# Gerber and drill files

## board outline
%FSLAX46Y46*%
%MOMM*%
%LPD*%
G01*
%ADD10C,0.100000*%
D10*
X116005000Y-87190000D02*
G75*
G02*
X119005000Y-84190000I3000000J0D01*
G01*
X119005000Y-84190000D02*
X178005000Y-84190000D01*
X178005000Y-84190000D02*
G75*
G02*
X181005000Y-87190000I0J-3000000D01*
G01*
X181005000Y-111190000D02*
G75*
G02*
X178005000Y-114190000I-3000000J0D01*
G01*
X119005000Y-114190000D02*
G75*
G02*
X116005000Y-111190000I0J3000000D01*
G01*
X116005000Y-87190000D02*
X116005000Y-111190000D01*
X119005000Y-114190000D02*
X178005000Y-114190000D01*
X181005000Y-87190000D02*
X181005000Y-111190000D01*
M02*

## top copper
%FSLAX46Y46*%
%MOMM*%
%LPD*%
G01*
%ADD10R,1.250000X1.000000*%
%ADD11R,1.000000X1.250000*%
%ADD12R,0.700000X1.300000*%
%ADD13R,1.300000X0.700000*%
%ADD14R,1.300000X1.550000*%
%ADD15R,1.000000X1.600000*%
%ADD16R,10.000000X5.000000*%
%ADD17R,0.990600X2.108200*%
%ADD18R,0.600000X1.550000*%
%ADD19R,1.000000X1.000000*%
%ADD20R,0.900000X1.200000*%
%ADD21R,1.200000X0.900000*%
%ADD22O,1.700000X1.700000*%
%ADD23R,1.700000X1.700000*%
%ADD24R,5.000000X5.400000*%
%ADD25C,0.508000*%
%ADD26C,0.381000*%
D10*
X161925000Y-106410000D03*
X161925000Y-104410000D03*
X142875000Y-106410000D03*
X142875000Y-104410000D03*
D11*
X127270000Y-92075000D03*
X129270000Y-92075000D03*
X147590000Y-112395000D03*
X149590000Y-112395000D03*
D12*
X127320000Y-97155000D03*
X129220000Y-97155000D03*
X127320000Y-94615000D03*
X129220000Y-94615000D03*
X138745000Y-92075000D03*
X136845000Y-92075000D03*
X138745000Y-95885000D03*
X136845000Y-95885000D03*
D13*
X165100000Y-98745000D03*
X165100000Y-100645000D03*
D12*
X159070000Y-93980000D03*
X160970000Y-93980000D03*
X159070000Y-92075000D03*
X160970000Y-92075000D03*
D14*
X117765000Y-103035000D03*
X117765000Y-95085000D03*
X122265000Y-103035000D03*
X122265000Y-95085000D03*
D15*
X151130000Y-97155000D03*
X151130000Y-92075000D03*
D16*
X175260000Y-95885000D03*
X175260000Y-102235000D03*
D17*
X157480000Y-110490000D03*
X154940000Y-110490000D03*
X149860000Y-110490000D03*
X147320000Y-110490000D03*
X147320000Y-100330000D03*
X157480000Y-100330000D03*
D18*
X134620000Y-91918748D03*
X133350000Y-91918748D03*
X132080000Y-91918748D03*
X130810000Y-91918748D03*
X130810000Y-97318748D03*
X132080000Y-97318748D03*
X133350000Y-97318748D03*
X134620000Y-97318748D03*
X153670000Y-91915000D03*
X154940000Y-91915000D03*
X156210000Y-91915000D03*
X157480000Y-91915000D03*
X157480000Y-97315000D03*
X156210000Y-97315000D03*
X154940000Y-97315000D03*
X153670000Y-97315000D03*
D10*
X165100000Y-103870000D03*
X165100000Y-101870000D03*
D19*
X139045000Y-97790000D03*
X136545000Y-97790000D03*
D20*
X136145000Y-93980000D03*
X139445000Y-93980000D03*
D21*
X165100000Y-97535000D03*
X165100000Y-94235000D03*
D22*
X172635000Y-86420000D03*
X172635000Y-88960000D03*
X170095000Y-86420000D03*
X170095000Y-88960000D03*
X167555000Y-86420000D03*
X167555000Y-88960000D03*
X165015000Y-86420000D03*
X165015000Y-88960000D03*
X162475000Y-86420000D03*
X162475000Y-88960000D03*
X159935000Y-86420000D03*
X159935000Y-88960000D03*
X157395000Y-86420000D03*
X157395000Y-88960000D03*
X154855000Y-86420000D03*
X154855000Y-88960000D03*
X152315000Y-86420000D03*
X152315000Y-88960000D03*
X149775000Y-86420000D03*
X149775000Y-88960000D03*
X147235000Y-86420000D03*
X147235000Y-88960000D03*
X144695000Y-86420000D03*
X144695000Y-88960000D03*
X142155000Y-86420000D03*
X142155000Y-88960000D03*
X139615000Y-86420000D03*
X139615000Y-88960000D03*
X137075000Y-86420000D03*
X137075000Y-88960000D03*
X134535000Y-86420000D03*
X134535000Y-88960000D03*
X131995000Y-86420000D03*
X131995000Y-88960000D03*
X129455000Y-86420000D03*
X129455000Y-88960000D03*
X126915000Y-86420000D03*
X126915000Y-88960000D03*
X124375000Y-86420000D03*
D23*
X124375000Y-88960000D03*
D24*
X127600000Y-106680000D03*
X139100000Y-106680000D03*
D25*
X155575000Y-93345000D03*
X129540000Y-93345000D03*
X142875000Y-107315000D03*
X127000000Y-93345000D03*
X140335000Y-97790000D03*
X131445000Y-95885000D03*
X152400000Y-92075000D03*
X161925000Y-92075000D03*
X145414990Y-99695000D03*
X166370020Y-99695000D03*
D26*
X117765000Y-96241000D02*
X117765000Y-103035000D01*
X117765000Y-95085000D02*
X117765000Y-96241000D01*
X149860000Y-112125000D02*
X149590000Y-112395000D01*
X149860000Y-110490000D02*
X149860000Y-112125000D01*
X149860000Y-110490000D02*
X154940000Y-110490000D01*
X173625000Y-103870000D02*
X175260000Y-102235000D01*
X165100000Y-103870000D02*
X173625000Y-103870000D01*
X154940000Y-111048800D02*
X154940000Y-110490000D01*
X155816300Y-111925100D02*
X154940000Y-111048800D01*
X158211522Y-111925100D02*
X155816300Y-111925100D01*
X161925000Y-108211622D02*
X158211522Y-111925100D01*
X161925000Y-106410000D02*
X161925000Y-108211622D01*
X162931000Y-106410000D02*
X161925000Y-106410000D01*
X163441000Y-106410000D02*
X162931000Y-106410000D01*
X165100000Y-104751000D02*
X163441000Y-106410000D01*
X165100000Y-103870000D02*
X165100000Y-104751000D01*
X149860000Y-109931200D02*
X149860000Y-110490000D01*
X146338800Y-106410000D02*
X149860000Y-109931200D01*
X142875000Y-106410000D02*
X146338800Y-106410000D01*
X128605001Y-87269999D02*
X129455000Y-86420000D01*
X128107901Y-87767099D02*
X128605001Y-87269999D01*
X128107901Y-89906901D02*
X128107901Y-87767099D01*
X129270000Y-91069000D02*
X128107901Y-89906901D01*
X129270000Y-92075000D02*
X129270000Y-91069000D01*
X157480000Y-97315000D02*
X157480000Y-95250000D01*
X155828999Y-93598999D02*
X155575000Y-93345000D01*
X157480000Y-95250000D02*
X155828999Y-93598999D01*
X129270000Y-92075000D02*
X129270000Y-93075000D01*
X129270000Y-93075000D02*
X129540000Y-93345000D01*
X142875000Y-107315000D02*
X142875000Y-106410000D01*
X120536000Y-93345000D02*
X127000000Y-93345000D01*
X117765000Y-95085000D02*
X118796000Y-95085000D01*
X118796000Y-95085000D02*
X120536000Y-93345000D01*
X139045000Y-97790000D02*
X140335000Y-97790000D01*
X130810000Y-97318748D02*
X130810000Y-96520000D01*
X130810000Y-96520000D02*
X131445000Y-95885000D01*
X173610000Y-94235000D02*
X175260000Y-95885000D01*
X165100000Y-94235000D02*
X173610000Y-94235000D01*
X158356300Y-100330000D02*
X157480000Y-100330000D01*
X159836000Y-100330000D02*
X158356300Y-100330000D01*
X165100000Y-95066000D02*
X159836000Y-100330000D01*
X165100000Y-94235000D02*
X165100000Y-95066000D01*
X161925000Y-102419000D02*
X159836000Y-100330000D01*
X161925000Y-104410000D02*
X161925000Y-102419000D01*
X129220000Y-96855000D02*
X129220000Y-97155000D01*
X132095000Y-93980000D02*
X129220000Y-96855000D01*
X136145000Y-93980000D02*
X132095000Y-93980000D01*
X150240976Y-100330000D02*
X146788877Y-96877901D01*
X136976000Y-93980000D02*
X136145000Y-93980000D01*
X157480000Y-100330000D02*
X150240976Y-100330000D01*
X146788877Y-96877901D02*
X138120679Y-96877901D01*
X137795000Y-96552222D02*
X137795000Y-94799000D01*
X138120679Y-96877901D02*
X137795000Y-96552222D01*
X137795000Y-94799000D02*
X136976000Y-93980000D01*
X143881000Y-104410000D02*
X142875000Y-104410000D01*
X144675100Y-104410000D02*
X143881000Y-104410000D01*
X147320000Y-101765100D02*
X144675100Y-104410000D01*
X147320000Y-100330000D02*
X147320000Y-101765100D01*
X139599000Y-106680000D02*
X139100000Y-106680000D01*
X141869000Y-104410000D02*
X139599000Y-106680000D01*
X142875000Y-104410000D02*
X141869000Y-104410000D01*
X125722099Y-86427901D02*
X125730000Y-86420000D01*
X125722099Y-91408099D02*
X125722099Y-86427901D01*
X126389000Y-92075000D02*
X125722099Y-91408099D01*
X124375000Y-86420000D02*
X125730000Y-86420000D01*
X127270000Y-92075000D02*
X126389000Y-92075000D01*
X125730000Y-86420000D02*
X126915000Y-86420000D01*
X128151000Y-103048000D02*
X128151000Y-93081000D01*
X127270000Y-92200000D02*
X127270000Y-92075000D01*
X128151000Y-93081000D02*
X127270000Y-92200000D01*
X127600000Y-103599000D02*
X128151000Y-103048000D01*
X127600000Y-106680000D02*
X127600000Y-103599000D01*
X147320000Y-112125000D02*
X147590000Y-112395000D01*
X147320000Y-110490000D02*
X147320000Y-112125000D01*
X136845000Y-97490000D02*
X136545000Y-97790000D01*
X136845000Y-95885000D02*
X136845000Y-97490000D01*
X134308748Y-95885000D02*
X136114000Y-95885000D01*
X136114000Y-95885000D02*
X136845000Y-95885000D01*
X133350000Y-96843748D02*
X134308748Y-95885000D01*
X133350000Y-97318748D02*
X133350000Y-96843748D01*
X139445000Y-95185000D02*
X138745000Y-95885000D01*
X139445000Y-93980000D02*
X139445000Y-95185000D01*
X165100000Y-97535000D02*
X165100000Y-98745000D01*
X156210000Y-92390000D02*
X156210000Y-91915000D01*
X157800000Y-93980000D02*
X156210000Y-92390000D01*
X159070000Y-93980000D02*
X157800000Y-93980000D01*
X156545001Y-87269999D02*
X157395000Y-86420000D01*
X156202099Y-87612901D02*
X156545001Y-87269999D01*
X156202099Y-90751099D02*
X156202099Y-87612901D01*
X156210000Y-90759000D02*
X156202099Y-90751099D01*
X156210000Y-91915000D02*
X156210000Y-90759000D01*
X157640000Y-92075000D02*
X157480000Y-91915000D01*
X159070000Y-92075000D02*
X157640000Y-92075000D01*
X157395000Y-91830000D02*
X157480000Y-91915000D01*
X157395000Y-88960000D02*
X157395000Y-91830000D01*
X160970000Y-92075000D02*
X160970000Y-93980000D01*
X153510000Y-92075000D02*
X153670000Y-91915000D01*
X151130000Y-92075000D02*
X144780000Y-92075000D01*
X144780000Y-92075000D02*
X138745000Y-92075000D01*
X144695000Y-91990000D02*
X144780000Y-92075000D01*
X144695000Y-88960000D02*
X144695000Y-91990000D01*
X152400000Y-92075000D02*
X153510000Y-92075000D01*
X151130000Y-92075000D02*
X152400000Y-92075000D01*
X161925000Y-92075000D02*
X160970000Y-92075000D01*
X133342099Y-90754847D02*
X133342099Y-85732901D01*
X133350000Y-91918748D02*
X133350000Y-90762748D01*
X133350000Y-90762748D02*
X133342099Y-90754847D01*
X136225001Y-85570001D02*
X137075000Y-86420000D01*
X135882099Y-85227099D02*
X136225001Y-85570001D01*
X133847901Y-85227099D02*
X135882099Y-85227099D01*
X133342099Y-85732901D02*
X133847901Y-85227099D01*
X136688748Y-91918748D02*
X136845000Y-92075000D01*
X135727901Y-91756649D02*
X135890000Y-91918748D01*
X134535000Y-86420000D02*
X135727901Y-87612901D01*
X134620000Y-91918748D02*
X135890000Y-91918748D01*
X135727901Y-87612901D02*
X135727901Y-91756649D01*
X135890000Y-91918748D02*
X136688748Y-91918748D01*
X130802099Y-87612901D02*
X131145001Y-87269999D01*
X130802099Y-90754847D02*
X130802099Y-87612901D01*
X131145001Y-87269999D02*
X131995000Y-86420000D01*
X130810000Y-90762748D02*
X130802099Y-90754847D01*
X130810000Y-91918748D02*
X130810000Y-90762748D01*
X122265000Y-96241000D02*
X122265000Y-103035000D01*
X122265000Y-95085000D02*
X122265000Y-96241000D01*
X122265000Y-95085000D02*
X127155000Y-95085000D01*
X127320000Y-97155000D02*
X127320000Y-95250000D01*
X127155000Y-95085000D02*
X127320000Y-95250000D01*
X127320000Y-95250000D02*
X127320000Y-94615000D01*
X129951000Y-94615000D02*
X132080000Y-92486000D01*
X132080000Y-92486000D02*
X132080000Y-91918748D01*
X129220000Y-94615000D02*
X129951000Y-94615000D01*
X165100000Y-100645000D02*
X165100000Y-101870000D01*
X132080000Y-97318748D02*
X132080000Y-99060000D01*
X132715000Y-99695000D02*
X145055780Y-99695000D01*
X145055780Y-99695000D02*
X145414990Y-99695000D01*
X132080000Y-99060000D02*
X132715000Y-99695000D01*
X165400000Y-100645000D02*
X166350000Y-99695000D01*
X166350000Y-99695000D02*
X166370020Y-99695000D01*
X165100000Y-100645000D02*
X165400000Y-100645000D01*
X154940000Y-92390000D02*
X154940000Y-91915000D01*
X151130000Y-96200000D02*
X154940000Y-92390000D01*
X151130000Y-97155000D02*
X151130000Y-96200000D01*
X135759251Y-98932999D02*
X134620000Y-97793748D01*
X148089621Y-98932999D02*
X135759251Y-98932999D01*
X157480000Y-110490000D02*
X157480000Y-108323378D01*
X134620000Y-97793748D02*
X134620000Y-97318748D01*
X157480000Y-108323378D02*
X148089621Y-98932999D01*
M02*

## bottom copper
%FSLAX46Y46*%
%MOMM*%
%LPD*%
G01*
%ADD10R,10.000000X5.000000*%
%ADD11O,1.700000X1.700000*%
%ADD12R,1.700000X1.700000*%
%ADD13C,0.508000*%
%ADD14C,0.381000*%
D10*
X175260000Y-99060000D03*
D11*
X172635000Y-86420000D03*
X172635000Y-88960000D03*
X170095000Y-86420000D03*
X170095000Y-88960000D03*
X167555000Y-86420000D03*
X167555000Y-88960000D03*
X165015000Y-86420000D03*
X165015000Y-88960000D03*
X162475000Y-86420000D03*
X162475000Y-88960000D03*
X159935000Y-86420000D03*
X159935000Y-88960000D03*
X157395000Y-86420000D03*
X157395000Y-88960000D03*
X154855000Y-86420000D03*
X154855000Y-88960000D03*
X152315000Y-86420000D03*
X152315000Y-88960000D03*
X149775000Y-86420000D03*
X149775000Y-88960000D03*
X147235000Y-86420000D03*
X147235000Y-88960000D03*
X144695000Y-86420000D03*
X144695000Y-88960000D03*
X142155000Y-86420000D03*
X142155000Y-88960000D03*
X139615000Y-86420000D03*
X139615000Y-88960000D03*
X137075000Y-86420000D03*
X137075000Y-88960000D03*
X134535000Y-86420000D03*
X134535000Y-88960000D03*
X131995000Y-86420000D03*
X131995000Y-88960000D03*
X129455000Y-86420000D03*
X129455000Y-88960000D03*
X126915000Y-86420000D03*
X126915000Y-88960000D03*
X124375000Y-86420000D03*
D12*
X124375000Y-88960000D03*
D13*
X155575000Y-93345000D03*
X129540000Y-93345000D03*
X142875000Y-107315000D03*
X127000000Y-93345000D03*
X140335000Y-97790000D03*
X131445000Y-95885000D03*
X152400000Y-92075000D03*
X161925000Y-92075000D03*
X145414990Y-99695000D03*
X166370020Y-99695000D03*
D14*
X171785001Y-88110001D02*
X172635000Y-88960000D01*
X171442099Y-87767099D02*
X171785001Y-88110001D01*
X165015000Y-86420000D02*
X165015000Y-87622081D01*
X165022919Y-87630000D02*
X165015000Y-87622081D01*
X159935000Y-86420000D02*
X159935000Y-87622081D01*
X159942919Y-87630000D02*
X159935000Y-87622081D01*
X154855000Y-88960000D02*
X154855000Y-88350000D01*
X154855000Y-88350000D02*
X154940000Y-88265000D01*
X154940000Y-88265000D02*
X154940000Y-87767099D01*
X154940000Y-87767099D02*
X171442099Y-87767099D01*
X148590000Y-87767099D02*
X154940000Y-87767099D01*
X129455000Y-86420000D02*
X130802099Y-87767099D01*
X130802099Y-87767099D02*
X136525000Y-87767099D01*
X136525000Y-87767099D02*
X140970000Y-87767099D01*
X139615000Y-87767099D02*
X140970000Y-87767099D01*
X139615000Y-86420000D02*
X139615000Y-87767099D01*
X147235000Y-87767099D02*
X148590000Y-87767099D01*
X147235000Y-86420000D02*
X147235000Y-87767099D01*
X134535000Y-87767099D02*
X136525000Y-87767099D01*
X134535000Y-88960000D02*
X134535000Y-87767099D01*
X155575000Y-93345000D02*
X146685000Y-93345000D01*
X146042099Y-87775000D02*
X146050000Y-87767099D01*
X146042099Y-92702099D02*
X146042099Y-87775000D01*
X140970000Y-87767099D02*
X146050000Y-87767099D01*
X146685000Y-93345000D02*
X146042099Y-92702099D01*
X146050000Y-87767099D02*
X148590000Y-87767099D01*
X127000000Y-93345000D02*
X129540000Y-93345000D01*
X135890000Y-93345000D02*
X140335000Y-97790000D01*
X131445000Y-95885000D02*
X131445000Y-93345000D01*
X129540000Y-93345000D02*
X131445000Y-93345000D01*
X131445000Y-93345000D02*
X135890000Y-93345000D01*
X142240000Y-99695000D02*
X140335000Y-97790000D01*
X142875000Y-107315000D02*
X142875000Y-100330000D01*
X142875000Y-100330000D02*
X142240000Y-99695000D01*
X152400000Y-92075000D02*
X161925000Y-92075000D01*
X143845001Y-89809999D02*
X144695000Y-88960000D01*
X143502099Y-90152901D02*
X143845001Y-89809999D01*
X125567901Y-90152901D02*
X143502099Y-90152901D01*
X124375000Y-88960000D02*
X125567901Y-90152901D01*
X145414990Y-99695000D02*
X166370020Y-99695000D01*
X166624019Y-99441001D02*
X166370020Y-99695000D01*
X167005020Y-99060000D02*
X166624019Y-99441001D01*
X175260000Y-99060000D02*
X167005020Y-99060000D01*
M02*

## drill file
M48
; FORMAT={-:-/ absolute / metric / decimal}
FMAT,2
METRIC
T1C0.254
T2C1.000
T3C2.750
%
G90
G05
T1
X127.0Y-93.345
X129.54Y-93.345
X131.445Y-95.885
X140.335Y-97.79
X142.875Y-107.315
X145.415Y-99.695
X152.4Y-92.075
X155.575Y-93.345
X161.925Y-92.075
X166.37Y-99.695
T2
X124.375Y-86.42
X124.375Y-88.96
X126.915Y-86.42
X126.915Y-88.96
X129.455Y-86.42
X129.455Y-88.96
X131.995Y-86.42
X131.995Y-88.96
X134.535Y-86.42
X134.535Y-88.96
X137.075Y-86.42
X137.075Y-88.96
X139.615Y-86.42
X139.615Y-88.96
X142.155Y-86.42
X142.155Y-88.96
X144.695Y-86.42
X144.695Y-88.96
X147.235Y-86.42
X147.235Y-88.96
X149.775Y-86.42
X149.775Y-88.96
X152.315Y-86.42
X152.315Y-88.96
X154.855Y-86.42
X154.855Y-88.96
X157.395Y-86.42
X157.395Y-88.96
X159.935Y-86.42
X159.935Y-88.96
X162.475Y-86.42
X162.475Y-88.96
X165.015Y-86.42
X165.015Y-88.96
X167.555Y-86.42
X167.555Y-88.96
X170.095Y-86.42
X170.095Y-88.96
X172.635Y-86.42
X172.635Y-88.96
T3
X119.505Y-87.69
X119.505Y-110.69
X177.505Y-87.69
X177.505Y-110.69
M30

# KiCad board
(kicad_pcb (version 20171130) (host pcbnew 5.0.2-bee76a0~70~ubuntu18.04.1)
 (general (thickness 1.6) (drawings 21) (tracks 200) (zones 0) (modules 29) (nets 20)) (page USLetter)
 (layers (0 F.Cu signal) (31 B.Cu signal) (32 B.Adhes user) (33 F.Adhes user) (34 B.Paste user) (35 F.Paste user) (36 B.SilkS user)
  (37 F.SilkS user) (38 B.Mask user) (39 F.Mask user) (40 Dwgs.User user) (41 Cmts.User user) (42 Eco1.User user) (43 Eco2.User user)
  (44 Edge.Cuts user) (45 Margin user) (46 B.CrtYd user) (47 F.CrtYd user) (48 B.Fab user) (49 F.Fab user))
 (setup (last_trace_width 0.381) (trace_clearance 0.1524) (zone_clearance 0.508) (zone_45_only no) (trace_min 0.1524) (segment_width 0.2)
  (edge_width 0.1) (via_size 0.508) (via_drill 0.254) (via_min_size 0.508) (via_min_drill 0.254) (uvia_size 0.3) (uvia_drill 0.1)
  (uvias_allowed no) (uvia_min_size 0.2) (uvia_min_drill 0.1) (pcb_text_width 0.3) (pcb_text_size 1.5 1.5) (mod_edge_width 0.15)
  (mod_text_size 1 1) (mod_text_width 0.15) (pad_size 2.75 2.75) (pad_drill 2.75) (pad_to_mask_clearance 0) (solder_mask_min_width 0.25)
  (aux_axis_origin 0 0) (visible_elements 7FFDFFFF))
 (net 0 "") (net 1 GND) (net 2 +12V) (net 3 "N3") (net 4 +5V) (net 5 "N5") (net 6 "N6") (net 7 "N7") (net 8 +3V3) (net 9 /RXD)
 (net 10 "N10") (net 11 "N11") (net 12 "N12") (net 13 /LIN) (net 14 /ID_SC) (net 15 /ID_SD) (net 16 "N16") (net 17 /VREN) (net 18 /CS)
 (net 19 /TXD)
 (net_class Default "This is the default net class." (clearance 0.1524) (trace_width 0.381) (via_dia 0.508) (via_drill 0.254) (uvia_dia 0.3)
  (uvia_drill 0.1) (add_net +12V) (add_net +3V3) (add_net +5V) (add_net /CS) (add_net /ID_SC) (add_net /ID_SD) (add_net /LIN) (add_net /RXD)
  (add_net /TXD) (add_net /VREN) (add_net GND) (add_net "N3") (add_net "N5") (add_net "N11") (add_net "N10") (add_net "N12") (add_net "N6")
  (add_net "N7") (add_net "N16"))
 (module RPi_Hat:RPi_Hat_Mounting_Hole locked (layer F.Cu) (at 119.505 110.69)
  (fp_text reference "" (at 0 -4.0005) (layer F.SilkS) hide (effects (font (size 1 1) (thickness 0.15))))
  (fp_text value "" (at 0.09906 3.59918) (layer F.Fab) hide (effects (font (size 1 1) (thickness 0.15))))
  (pad "" np_thru_hole circle (at 0 0) (size 2.75 2.75) (drill 2.75) (layers *.Cu *.Mask) (solder_mask_margin 1.725) (clearance 1.725)))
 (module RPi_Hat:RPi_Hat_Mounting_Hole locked (layer F.Cu) (at 177.505 87.69)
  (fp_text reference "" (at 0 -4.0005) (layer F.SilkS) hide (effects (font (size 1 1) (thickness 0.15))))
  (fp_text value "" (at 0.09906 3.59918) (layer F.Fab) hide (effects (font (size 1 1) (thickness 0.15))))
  (pad "" np_thru_hole circle (at 0 0) (size 2.75 2.75) (drill 2.75) (layers *.Cu *.Mask) (solder_mask_margin 1.725) (clearance 1.725)))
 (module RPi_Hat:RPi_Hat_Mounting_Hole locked (layer F.Cu) (at 177.505 110.69)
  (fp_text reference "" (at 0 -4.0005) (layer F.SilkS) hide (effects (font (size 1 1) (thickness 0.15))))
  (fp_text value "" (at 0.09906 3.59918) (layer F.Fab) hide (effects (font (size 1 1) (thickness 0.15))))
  (pad "" np_thru_hole circle (at 0 0) (size 2.75 2.75) (drill 2.75) (layers *.Cu *.Mask) (solder_mask_margin 1.725) (clearance 1.725)))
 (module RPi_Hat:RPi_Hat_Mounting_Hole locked (layer F.Cu) (at 119.505 87.69)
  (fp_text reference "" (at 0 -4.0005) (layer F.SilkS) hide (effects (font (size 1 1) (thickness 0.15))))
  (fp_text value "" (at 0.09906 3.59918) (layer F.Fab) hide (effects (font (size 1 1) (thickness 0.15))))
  (pad "" np_thru_hole circle (at 0 0) (size 2.75 2.75) (drill 2.75) (layers *.Cu *.Mask) (solder_mask_margin 1.725) (clearance 1.725)))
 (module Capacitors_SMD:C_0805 (layer F.Cu) (at 161.925 105.41 270)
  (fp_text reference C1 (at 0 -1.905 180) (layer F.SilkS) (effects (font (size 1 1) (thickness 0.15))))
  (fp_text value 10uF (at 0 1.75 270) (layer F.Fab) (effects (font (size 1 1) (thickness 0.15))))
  (pad 2 smd rect (at 1 0 270) (size 1 1.25) (layers F.Cu F.Paste F.Mask) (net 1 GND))
  (pad 1 smd rect (at -1 0 270) (size 1 1.25) (layers F.Cu F.Paste F.Mask) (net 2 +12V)))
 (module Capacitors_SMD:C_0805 (layer F.Cu) (at 142.875 105.41 270)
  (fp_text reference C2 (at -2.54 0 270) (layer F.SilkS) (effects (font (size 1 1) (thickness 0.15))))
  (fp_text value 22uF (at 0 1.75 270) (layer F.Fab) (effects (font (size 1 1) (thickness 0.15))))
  (pad 2 smd rect (at 1 0 270) (size 1 1.25) (layers F.Cu F.Paste F.Mask) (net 1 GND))
  (pad 1 smd rect (at -1 0 270) (size 1 1.25) (layers F.Cu F.Paste F.Mask) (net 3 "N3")))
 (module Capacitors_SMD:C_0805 (layer F.Cu) (at 128.27 92.075)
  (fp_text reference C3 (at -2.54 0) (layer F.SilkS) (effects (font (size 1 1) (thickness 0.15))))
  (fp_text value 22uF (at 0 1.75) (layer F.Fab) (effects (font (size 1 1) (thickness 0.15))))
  (pad 1 smd rect (at -1 0) (size 1 1.25) (layers F.Cu F.Paste F.Mask) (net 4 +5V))
  (pad 2 smd rect (at 1 0) (size 1 1.25) (layers F.Cu F.Paste F.Mask) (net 1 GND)))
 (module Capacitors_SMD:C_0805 (layer F.Cu) (at 148.59 112.395)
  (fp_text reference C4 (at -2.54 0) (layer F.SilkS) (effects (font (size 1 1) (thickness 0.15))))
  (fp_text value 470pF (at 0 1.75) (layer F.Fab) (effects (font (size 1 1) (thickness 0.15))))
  (pad 1 smd rect (at -1 0) (size 1 1.25) (layers F.Cu F.Paste F.Mask) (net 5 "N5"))
  (pad 2 smd rect (at 1 0) (size 1 1.25) (layers F.Cu F.Paste F.Mask) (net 1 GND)))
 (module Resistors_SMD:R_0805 (layer F.Cu) (at 128.27 97.155 180)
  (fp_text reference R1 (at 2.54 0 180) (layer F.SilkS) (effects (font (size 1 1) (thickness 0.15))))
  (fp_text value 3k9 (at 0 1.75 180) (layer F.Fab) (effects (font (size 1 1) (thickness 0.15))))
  (pad 2 smd rect (at 0.95 0 180) (size 0.7 1.3) (layers F.Cu F.Paste F.Mask) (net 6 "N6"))
  (pad 1 smd rect (at -0.95 0 180) (size 0.7 1.3) (layers F.Cu F.Paste F.Mask) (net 2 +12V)))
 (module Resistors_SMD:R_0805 (layer F.Cu) (at 128.27 94.615 180)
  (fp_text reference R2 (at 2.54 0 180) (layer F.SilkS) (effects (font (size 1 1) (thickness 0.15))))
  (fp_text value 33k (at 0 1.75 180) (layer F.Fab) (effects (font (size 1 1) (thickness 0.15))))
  (pad 2 smd rect (at 0.95 0 180) (size 0.7 1.3) (layers F.Cu F.Paste F.Mask) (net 6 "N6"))
  (pad 1 smd rect (at -0.95 0 180) (size 0.7 1.3) (layers F.Cu F.Paste F.Mask) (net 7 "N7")))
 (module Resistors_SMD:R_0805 (layer F.Cu) (at 137.795 92.075 180)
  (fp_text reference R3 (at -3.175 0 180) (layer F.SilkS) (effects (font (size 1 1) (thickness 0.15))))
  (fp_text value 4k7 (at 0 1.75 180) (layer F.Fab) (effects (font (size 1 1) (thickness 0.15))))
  (pad 1 smd rect (at -0.95 0 180) (size 0.7 1.3) (layers F.Cu F.Paste F.Mask) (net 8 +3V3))
  (pad 2 smd rect (at 0.95 0 180) (size 0.7 1.3) (layers F.Cu F.Paste F.Mask) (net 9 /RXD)))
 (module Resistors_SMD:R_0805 (layer F.Cu) (at 137.795 95.885 180)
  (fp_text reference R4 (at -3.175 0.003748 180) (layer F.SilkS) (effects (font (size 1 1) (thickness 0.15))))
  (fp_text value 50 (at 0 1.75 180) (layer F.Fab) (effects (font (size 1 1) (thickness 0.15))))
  (pad 1 smd rect (at -0.95 0 180) (size 0.7 1.3) (layers F.Cu F.Paste F.Mask) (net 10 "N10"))
  (pad 2 smd rect (at 0.95 0 180) (size 0.7 1.3) (layers F.Cu F.Paste F.Mask) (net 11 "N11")))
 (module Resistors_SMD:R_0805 (layer F.Cu) (at 165.1 99.695 270)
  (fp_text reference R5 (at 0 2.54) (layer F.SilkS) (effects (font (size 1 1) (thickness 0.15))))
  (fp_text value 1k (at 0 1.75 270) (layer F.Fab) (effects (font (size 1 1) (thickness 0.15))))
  (pad 1 smd rect (at -0.95 0 270) (size 0.7 1.3) (layers F.Cu F.Paste F.Mask) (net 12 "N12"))
  (pad 2 smd rect (at 0.95 0 270) (size 0.7 1.3) (layers F.Cu F.Paste F.Mask) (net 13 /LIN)))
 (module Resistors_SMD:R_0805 (layer F.Cu) (at 160.02 93.98 180)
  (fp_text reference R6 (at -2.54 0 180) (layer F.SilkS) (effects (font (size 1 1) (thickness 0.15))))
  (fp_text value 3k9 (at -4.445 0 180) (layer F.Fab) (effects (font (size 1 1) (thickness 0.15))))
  (pad 2 smd rect (at 0.95 0 180) (size 0.7 1.3) (layers F.Cu F.Paste F.Mask) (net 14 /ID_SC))
  (pad 1 smd rect (at -0.95 0 180) (size 0.7 1.3) (layers F.Cu F.Paste F.Mask) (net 8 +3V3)))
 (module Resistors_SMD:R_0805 (layer F.Cu) (at 160.02 92.075 180)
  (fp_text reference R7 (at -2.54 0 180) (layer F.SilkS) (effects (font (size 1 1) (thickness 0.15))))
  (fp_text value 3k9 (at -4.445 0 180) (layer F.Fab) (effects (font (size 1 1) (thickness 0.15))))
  (pad 2 smd rect (at 0.95 0 180) (size 0.7 1.3) (layers F.Cu F.Paste F.Mask) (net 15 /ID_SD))
  (pad 1 smd rect (at -0.95 0 180) (size 0.7 1.3) (layers F.Cu F.Paste F.Mask) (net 8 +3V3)))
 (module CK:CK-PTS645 (layer F.Cu) (at 120.015 99.06 270)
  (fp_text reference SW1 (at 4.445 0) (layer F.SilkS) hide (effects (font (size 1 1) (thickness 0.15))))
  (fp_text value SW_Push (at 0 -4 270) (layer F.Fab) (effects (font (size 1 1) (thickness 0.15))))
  (pad 2 smd rect (at 3.975 2.25 270) (size 1.55 1.3) (layers F.Cu F.Paste F.Mask) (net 1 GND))
  (pad 2 smd rect (at -3.975 2.25 270) (size 1.55 1.3) (layers F.Cu F.Paste F.Mask) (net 1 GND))
  (pad 1 smd rect (at 3.975 -2.25 270) (size 1.55 1.3) (layers F.Cu F.Paste F.Mask) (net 6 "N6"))
  (pad 1 smd rect (at -3.975 -2.25 270) (size 1.55 1.3) (layers F.Cu F.Paste F.Mask) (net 6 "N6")))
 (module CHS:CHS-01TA (layer F.Cu) (at 151.13 94.615)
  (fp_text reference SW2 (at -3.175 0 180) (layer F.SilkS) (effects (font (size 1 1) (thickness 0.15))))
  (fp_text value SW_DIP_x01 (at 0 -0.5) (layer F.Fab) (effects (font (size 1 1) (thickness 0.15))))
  (pad 2 smd rect (at 0 2.54) (size 1 1.6) (layers F.Cu F.Paste F.Mask) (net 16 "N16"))
  (pad 1 smd rect (at 0 -2.54) (size 1 1.6) (layers F.Cu F.Paste F.Mask) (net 8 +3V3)))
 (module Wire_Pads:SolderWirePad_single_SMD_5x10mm (layer F.Cu) (at 175.26 95.885 90)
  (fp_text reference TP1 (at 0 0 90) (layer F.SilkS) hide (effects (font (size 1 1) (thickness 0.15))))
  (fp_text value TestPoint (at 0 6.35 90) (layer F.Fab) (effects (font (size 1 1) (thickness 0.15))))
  (pad 1 smd rect (at 0 0 90) (size 5 10) (layers F.Cu F.Paste F.Mask) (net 2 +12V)))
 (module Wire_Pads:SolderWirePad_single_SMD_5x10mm (layer B.Cu) (at 175.26 99.06 270)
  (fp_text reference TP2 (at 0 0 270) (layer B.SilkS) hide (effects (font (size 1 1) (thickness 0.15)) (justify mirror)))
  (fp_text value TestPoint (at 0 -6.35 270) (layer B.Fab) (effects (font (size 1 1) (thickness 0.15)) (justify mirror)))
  (pad 1 smd rect (at 0 0 270) (size 5 10) (layers B.Cu B.Paste B.Mask) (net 13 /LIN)))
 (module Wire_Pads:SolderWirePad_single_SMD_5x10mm (layer F.Cu) (at 175.26 102.235 270)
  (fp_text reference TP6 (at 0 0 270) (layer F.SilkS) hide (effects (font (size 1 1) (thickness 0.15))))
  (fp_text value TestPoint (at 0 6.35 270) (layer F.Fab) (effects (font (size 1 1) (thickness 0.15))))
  (pad 1 smd rect (at 0 0 270) (size 5 10) (layers F.Cu F.Paste F.Mask) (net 1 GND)))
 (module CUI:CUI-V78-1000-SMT (layer F.Cu) (at 157.48 100.33 180)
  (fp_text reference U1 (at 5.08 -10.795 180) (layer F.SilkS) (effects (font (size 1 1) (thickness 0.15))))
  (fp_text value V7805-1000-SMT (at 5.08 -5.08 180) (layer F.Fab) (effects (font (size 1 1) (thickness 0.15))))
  (pad 10 smd rect (at 0 -10.16 180) (size 0.9906 2.1082) (layers F.Cu F.Paste F.Mask) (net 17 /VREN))
  (pad 9 smd rect (at 2.54 -10.16 180) (size 0.9906 2.1082) (layers F.Cu F.Paste F.Mask) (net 1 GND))
  (pad 7 smd rect (at 7.62 -10.16 180) (size 0.9906 2.1082) (layers F.Cu F.Paste F.Mask) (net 1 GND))
  (pad 6 smd rect (at 10.16 -10.16 180) (size 0.9906 2.1082) (layers F.Cu F.Paste F.Mask) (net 5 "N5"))
  (pad 5 smd rect (at 10.16 0 180) (size 0.9906 2.1082) (layers F.Cu F.Paste F.Mask) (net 3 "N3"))
  (pad 1 smd rect (at 0 0 180) (size 0.9906 2.1082) (layers F.Cu F.Paste F.Mask) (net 2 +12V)))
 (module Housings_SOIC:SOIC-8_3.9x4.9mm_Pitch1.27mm (layer F.Cu) (at 132.715 94.618748 270)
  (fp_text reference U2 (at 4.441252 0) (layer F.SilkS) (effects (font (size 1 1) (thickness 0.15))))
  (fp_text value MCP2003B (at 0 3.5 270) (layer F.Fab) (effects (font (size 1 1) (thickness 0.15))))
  (pad 1 smd rect (at -2.7 -1.905 270) (size 1.55 0.6) (layers F.Cu F.Paste F.Mask) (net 9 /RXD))
  (pad 2 smd rect (at -2.7 -0.635 270) (size 1.55 0.6) (layers F.Cu F.Paste F.Mask) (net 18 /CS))
  (pad 3 smd rect (at -2.7 0.635 270) (size 1.55 0.6) (layers F.Cu F.Paste F.Mask) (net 7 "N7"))
  (pad 4 smd rect (at -2.7 1.905 270) (size 1.55 0.6) (layers F.Cu F.Paste F.Mask) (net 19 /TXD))
  (pad 5 smd rect (at 2.7 1.905 270) (size 1.55 0.6) (layers F.Cu F.Paste F.Mask) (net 1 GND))
  (pad 6 smd rect (at 2.7 0.635 270) (size 1.55 0.6) (layers F.Cu F.Paste F.Mask) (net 13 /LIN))
  (pad 7 smd rect (at 2.7 -0.635 270) (size 1.55 0.6) (layers F.Cu F.Paste F.Mask) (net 11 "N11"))
  (pad 8 smd rect (at 2.7 -1.905 270) (size 1.55 0.6) (layers F.Cu F.Paste F.Mask) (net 17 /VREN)))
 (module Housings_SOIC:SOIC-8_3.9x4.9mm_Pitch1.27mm (layer F.Cu) (at 155.575 94.615 90)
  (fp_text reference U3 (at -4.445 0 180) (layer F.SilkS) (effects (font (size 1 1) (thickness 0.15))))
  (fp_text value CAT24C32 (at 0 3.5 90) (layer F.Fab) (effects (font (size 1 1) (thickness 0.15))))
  (pad 8 smd rect (at 2.7 -1.905 90) (size 1.55 0.6) (layers F.Cu F.Paste F.Mask) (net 8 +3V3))
  (pad 7 smd rect (at 2.7 -0.635 90) (size 1.55 0.6) (layers F.Cu F.Paste F.Mask) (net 16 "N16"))
  (pad 6 smd rect (at 2.7 0.635 90) (size 1.55 0.6) (layers F.Cu F.Paste F.Mask) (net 14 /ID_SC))
  (pad 5 smd rect (at 2.7 1.905 90) (size 1.55 0.6) (layers F.Cu F.Paste F.Mask) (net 15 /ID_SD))
  (pad 4 smd rect (at -2.7 1.905 90) (size 1.55 0.6) (layers F.Cu F.Paste F.Mask) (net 1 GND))
  (pad 3 smd rect (at -2.7 0.635 90) (size 1.55 0.6) (layers F.Cu F.Paste F.Mask))
  (pad 2 smd rect (at -2.7 -0.635 90) (size 1.55 0.6) (layers F.Cu F.Paste F.Mask))
  (pad 1 smd rect (at -2.7 -1.905 90) (size 1.55 0.6) (layers F.Cu F.Paste F.Mask)))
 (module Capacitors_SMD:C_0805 (layer F.Cu) (at 165.1 102.87 270)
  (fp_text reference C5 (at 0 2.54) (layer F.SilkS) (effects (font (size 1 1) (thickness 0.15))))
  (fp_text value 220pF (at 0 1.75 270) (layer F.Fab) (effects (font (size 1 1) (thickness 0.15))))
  (pad 2 smd rect (at 1 0 270) (size 1 1.25) (layers F.Cu F.Paste F.Mask) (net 1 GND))
  (pad 1 smd rect (at -1 0 270) (size 1 1.25) (layers F.Cu F.Paste F.Mask) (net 13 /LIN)))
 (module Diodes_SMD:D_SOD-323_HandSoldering (layer F.Cu) (at 137.795 97.79)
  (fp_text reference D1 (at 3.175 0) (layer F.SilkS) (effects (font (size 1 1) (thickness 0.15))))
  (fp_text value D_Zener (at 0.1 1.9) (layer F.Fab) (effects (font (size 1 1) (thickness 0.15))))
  (pad 2 smd rect (at 1.25 0) (size 1 1) (layers F.Cu F.Paste F.Mask) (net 1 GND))
  (pad 1 smd rect (at -1.25 0) (size 1 1) (layers F.Cu F.Paste F.Mask) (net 11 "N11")))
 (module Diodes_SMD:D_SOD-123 (layer F.Cu) (at 137.795 93.98 180)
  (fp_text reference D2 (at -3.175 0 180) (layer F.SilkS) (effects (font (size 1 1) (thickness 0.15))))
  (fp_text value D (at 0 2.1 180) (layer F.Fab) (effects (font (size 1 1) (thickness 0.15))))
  (pad 2 smd rect (at 1.65 0 180) (size 0.9 1.2) (layers F.Cu F.Paste F.Mask) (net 2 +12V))
  (pad 1 smd rect (at -1.65 0 180) (size 0.9 1.2) (layers F.Cu F.Paste F.Mask) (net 10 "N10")))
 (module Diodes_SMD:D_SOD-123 (layer F.Cu) (at 165.1 95.885 90)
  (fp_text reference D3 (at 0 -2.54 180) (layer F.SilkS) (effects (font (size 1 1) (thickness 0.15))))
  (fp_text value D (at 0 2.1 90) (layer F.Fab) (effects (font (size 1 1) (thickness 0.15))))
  (pad 1 smd rect (at -1.65 0 90) (size 0.9 1.2) (layers F.Cu F.Paste F.Mask) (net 12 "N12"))
  (pad 2 smd rect (at 1.65 0 90) (size 0.9 1.2) (layers F.Cu F.Paste F.Mask) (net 2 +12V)))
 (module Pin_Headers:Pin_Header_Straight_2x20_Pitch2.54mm (layer F.Cu) (at 124.375 88.96 90)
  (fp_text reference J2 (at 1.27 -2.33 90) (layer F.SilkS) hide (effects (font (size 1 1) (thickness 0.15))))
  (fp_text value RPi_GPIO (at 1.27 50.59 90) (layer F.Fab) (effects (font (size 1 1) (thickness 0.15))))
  (pad 40 thru_hole oval (at 2.54 48.26 90) (size 1.7 1.7) (drill 1) (layers *.Cu *.Mask))
  (pad 39 thru_hole oval (at 0 48.26 90) (size 1.7 1.7) (drill 1) (layers *.Cu *.Mask) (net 1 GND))
  (pad 38 thru_hole oval (at 2.54 45.72 90) (size 1.7 1.7) (drill 1) (layers *.Cu *.Mask))
  (pad 37 thru_hole oval (at 0 45.72 90) (size 1.7 1.7) (drill 1) (layers *.Cu *.Mask))
  (pad 36 thru_hole oval (at 2.54 43.18 90) (size 1.7 1.7) (drill 1) (layers *.Cu *.Mask))
  (pad 35 thru_hole oval (at 0 43.18 90) (size 1.7 1.7) (drill 1) (layers *.Cu *.Mask))
  (pad 34 thru_hole oval (at 2.54 40.64 90) (size 1.7 1.7) (drill 1) (layers *.Cu *.Mask) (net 1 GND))
  (pad 33 thru_hole oval (at 0 40.64 90) (size 1.7 1.7) (drill 1) (layers *.Cu *.Mask))
  (pad 32 thru_hole oval (at 2.54 38.1 90) (size 1.7 1.7) (drill 1) (layers *.Cu *.Mask))
  (pad 31 thru_hole oval (at 0 38.1 90) (size 1.7 1.7) (drill 1) (layers *.Cu *.Mask))
  (pad 30 thru_hole oval (at 2.54 35.56 90) (size 1.7 1.7) (drill 1) (layers *.Cu *.Mask) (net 1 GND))
  (pad 29 thru_hole oval (at 0 35.56 90) (size 1.7 1.7) (drill 1) (layers *.Cu *.Mask))
  (pad 28 thru_hole oval (at 2.54 33.02 90) (size 1.7 1.7) (drill 1) (layers *.Cu *.Mask) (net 14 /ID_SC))
  (pad 27 thru_hole oval (at 0 33.02 90) (size 1.7 1.7) (drill 1) (layers *.Cu *.Mask) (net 15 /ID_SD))
  (pad 26 thru_hole oval (at 2.54 30.48 90) (size 1.7 1.7) (drill 1) (layers *.Cu *.Mask))
  (pad 25 thru_hole oval (at 0 30.48 90) (size 1.7 1.7) (drill 1) (layers *.Cu *.Mask) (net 1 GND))
  (pad 24 thru_hole oval (at 2.54 27.94 90) (size 1.7 1.7) (drill 1) (layers *.Cu *.Mask))
  (pad 23 thru_hole oval (at 0 27.94 90) (size 1.7 1.7) (drill 1) (layers *.Cu *.Mask))
  (pad 22 thru_hole oval (at 2.54 25.4 90) (size 1.7 1.7) (drill 1) (layers *.Cu *.Mask))
  (pad 21 thru_hole oval (at 0 25.4 90) (size 1.7 1.7) (drill 1) (layers *.Cu *.Mask))
  (pad 20 thru_hole oval (at 2.54 22.86 90) (size 1.7 1.7) (drill 1) (layers *.Cu *.Mask) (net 1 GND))
  (pad 19 thru_hole oval (at 0 22.86 90) (size 1.7 1.7) (drill 1) (layers *.Cu *.Mask))
  (pad 18 thru_hole oval (at 2.54 20.32 90) (size 1.7 1.7) (drill 1) (layers *.Cu *.Mask))
  (pad 17 thru_hole oval (at 0 20.32 90) (size 1.7 1.7) (drill 1) (layers *.Cu *.Mask) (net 8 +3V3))
  (pad 16 thru_hole oval (at 2.54 17.78 90) (size 1.7 1.7) (drill 1) (layers *.Cu *.Mask))
  (pad 15 thru_hole oval (at 0 17.78 90) (size 1.7 1.7) (drill 1) (layers *.Cu *.Mask))
  (pad 14 thru_hole oval (at 2.54 15.24 90) (size 1.7 1.7) (drill 1) (layers *.Cu *.Mask) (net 1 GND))
  (pad 13 thru_hole oval (at 0 15.24 90) (size 1.7 1.7) (drill 1) (layers *.Cu *.Mask))
  (pad 12 thru_hole oval (at 2.54 12.7 90) (size 1.7 1.7) (drill 1) (layers *.Cu *.Mask) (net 18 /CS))
  (pad 11 thru_hole oval (at 0 12.7 90) (size 1.7 1.7) (drill 1) (layers *.Cu *.Mask))
  (pad 10 thru_hole oval (at 2.54 10.16 90) (size 1.7 1.7) (drill 1) (layers *.Cu *.Mask) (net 9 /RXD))
  (pad 9 thru_hole oval (at 0 10.16 90) (size 1.7 1.7) (drill 1) (layers *.Cu *.Mask) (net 1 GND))
  (pad 8 thru_hole oval (at 2.54 7.62 90) (size 1.7 1.7) (drill 1) (layers *.Cu *.Mask) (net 19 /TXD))
  (pad 7 thru_hole oval (at 0 7.62 90) (size 1.7 1.7) (drill 1) (layers *.Cu *.Mask))
  (pad 6 thru_hole oval (at 2.54 5.08 90) (size 1.7 1.7) (drill 1) (layers *.Cu *.Mask) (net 1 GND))
  (pad 5 thru_hole oval (at 0 5.08 90) (size 1.7 1.7) (drill 1) (layers *.Cu *.Mask))
  (pad 4 thru_hole oval (at 2.54 2.54 90) (size 1.7 1.7) (drill 1) (layers *.Cu *.Mask) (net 4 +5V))
  (pad 3 thru_hole oval (at 0 2.54 90) (size 1.7 1.7) (drill 1) (layers *.Cu *.Mask))
  (pad 2 thru_hole oval (at 2.54 0 90) (size 1.7 1.7) (drill 1) (layers *.Cu *.Mask) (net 4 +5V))
  (pad 1 thru_hole rect (at 0 0 90) (size 1.7 1.7) (drill 1) (layers *.Cu *.Mask) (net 8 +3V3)))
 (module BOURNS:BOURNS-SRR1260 (layer F.Cu) (at 133.35 106.68 180)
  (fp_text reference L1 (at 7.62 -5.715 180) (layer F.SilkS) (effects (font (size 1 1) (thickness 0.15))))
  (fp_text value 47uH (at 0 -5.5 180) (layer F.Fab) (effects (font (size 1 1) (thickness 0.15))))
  (pad 2 smd rect (at 5.75 0 180) (size 5 5.4) (layers F.Cu F.Paste F.Mask) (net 4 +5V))
  (pad 1 smd rect (at -5.75 0 180) (size 5 5.4) (layers F.Cu F.Paste F.Mask) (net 3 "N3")))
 (gr_arc (start 119.005 87.19) (end 116.005 87.19) (angle 90) (layer Edge.Cuts) (width 0.1))
 (gr_line (start 119.005 84.19) (end 178.005 84.19) (angle 90) (layer Edge.Cuts) (width 0.1))
 (gr_arc (start 178.005 87.19) (end 178.005 84.19) (angle 90) (layer Edge.Cuts) (width 0.1))
 (gr_arc (start 178.005 111.19) (end 181.005 111.19) (angle 90) (layer Edge.Cuts) (width 0.1))
 (gr_arc (start 119.005 111.19) (end 119.005 114.19) (angle 90) (layer Edge.Cuts) (width 0.1))
 (gr_line (start 116.005 87.19) (end 116.005 111.19) (layer Edge.Cuts) (width 0.1))
 (gr_line (start 119.005 114.19) (end 178.005 114.19) (angle 90) (layer Edge.Cuts) (width 0.1))
 (gr_line (start 181.005 87.19) (end 181.005 111.19) (angle 90) (layer Edge.Cuts) (width 0.1))
 (segment (start 117.765 96.241) (end 117.765 103.035) (width 0.381) (layer F.Cu) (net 1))
 (segment (start 117.765 95.085) (end 117.765 96.241) (width 0.381) (layer F.Cu) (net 1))
 (segment (start 149.86 112.125) (end 149.59 112.395) (width 0.381) (layer F.Cu) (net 1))
 (segment (start 149.86 110.49) (end 149.86 112.125) (width 0.381) (layer F.Cu) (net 1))
 (segment (start 149.86 110.49) (end 154.94 110.49) (width 0.381) (layer F.Cu) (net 1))
 (segment (start 173.625 103.87) (end 175.26 102.235) (width 0.381) (layer F.Cu) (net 1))
 (segment (start 165.1 103.87) (end 173.625 103.87) (width 0.381) (layer F.Cu) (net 1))
 (segment (start 154.94 111.0488) (end 154.94 110.49) (width 0.381) (layer F.Cu) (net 1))
 (segment (start 155.8163 111.9251) (end 154.94 111.0488) (width 0.381) (layer F.Cu) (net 1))
 (segment (start 158.211522 111.9251) (end 155.8163 111.9251) (width 0.381) (layer F.Cu) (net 1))
 (segment (start 161.925 108.211622) (end 158.211522 111.9251) (width 0.381) (layer F.Cu) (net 1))
 (segment (start 161.925 106.41) (end 161.925 108.211622) (width 0.381) (layer F.Cu) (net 1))
 (segment (start 162.931 106.41) (end 161.925 106.41) (width 0.381) (layer F.Cu) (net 1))
 (segment (start 163.441 106.41) (end 162.931 106.41) (width 0.381) (layer F.Cu) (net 1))
 (segment (start 165.1 104.751) (end 163.441 106.41) (width 0.381) (layer F.Cu) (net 1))
 (segment (start 165.1 103.87) (end 165.1 104.751) (width 0.381) (layer F.Cu) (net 1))
 (segment (start 149.86 109.9312) (end 149.86 110.49) (width 0.381) (layer F.Cu) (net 1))
 (segment (start 146.3388 106.41) (end 149.86 109.9312) (width 0.381) (layer F.Cu) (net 1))
 (segment (start 142.875 106.41) (end 146.3388 106.41) (width 0.381) (layer F.Cu) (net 1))
 (segment (start 171.785001 88.110001) (end 172.635 88.96) (width 0.381) (layer B.Cu) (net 1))
 (segment (start 171.442099 87.767099) (end 171.785001 88.110001) (width 0.381) (layer B.Cu) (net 1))
 (segment (start 165.015 86.42) (end 165.015 87.622081) (width 0.381) (layer B.Cu) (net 1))
 (segment (start 165.022919 87.63) (end 165.015 87.622081) (width 0.381) (layer B.Cu) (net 1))
 (segment (start 159.935 86.42) (end 159.935 87.622081) (width 0.381) (layer B.Cu) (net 1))
 (segment (start 159.942919 87.63) (end 159.935 87.622081) (width 0.381) (layer B.Cu) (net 1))
 (segment (start 154.855 88.96) (end 154.855 88.35) (width 0.381) (layer B.Cu) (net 1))
 (segment (start 154.855 88.35) (end 154.94 88.265) (width 0.381) (layer B.Cu) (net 1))
 (segment (start 154.94 88.265) (end 154.94 87.767099) (width 0.381) (layer B.Cu) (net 1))
 (segment (start 154.94 87.767099) (end 171.442099 87.767099) (width 0.381) (layer B.Cu) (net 1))
 (segment (start 148.59 87.767099) (end 154.94 87.767099) (width 0.381) (layer B.Cu) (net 1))
 (segment (start 129.455 86.42) (end 130.802099 87.767099) (width 0.381) (layer B.Cu) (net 1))
 (segment (start 130.802099 87.767099) (end 136.525 87.767099) (width 0.381) (layer B.Cu) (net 1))
 (segment (start 136.525 87.767099) (end 140.97 87.767099) (width 0.381) (layer B.Cu) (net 1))
 (segment (start 139.615 87.767099) (end 140.97 87.767099) (width 0.381) (layer B.Cu) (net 1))
 (segment (start 139.615 86.42) (end 139.615 87.767099) (width 0.381) (layer B.Cu) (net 1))
 (segment (start 147.235 87.767099) (end 148.59 87.767099) (width 0.381) (layer B.Cu) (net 1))
 (segment (start 147.235 86.42) (end 147.235 87.767099) (width 0.381) (layer B.Cu) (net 1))
 (segment (start 134.535 87.767099) (end 136.525 87.767099) (width 0.381) (layer B.Cu) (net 1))
 (segment (start 134.535 88.96) (end 134.535 87.767099) (width 0.381) (layer B.Cu) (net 1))
 (segment (start 128.605001 87.269999) (end 129.455 86.42) (width 0.381) (layer F.Cu) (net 1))
 (segment (start 128.107901 87.767099) (end 128.605001 87.269999) (width 0.381) (layer F.Cu) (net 1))
 (segment (start 128.107901 89.906901) (end 128.107901 87.767099) (width 0.381) (layer F.Cu) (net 1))
 (segment (start 129.27 91.069) (end 128.107901 89.906901) (width 0.381) (layer F.Cu) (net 1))
 (segment (start 129.27 92.075) (end 129.27 91.069) (width 0.381) (layer F.Cu) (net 1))
 (via (at 155.575 93.345) (size 0.508) (drill 0.254) (layers F.Cu B.Cu) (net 1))
 (segment (start 157.48 97.315) (end 157.48 95.25) (width 0.381) (layer F.Cu) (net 1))
 (segment (start 155.828999 93.598999) (end 155.575 93.345) (width 0.381) (layer F.Cu) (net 1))
 (segment (start 157.48 95.25) (end 155.828999 93.598999) (width 0.381) (layer F.Cu) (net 1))
 (segment (start 155.575 93.345) (end 146.685 93.345) (width 0.381) (layer B.Cu) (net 1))
 (segment (start 146.042099 87.775) (end 146.05 87.767099) (width 0.381) (layer B.Cu) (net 1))
 (segment (start 146.042099 92.702099) (end 146.042099 87.775) (width 0.381) (layer B.Cu) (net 1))
 (segment (start 140.97 87.767099) (end 146.05 87.767099) (width 0.381) (layer B.Cu) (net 1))
 (segment (start 146.685 93.345) (end 146.042099 92.702099) (width 0.381) (layer B.Cu) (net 1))
 (segment (start 146.05 87.767099) (end 148.59 87.767099) (width 0.381) (layer B.Cu) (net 1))
 (via (at 129.54 93.345) (size 0.508) (drill 0.254) (layers F.Cu B.Cu) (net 1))
 (segment (start 129.27 92.075) (end 129.27 93.075) (width 0.381) (layer F.Cu) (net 1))
 (segment (start 129.27 93.075) (end 129.54 93.345) (width 0.381) (layer F.Cu) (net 1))
 (via (at 142.875 107.315) (size 0.508) (drill 0.254) (layers F.Cu B.Cu) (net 1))
 (segment (start 142.875 107.315) (end 142.875 106.41) (width 0.381) (layer F.Cu) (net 1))
 (segment (start 120.536 93.345) (end 127 93.345) (width 0.381) (layer F.Cu) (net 1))
 (segment (start 117.765 95.085) (end 118.796 95.085) (width 0.381) (layer F.Cu) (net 1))
 (via (at 127 93.345) (size 0.508) (drill 0.254) (layers F.Cu B.Cu) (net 1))
 (segment (start 118.796 95.085) (end 120.536 93.345) (width 0.381) (layer F.Cu) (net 1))
 (segment (start 127 93.345) (end 129.54 93.345) (width 0.381) (layer B.Cu) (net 1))
 (via (at 140.335 97.79) (size 0.508) (drill 0.254) (layers F.Cu B.Cu) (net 1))
 (segment (start 139.045 97.79) (end 140.335 97.79) (width 0.381) (layer F.Cu) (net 1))
 (segment (start 135.89 93.345) (end 140.335 97.79) (width 0.381) (layer B.Cu) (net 1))
 (via (at 131.445 95.885) (size 0.508) (drill 0.254) (layers F.Cu B.Cu) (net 1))
 (segment (start 130.81 97.318748) (end 130.81 96.52) (width 0.381) (layer F.Cu) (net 1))
 (segment (start 130.81 96.52) (end 131.445 95.885) (width 0.381) (layer F.Cu) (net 1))
 (segment (start 131.445 95.885) (end 131.445 93.345) (width 0.381) (layer B.Cu) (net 1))
 (segment (start 129.54 93.345) (end 131.445 93.345) (width 0.381) (layer B.Cu) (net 1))
 (segment (start 131.445 93.345) (end 135.89 93.345) (width 0.381) (layer B.Cu) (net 1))
 (segment (start 142.24 99.695) (end 140.335 97.79) (width 0.381) (layer B.Cu) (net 1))
 (segment (start 142.875 107.315) (end 142.875 100.33) (width 0.381) (layer B.Cu) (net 1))
 (segment (start 142.875 100.33) (end 142.24 99.695) (width 0.381) (layer B.Cu) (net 1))
 (segment (start 173.61 94.235) (end 175.26 95.885) (width 0.381) (layer F.Cu) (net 2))
 (segment (start 165.1 94.235) (end 173.61 94.235) (width 0.381) (layer F.Cu) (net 2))
 (segment (start 158.3563 100.33) (end 157.48 100.33) (width 0.381) (layer F.Cu) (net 2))
 (segment (start 159.836 100.33) (end 158.3563 100.33) (width 0.381) (layer F.Cu) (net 2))
 (segment (start 165.1 95.066) (end 159.836 100.33) (width 0.381) (layer F.Cu) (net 2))
 (segment (start 165.1 94.235) (end 165.1 95.066) (width 0.381) (layer F.Cu) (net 2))
 (segment (start 161.925 102.419) (end 159.836 100.33) (width 0.381) (layer F.Cu) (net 2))
 (segment (start 161.925 104.41) (end 161.925 102.419) (width 0.381) (layer F.Cu) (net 2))
 (segment (start 129.22 96.855) (end 129.22 97.155) (width 0.381) (layer F.Cu) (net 2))
 (segment (start 132.095 93.98) (end 129.22 96.855) (width 0.381) (layer F.Cu) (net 2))
 (segment (start 136.145 93.98) (end 132.095 93.98) (width 0.381) (layer F.Cu) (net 2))
 (segment (start 150.240976 100.33) (end 146.788877 96.877901) (width 0.381) (layer F.Cu) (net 2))
 (segment (start 136.976 93.98) (end 136.145 93.98) (width 0.381) (layer F.Cu) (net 2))
 (segment (start 157.48 100.33) (end 150.240976 100.33) (width 0.381) (layer F.Cu) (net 2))
 (segment (start 146.788877 96.877901) (end 138.120679 96.877901) (width 0.381) (layer F.Cu) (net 2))
 (segment (start 137.795 96.552222) (end 137.795 94.799) (width 0.381) (layer F.Cu) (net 2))
 (segment (start 138.120679 96.877901) (end 137.795 96.552222) (width 0.381) (layer F.Cu) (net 2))
 (segment (start 137.795 94.799) (end 136.976 93.98) (width 0.381) (layer F.Cu) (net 2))
 (segment (start 143.881 104.41) (end 142.875 104.41) (width 0.381) (layer F.Cu) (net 3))
 (segment (start 144.6751 104.41) (end 143.881 104.41) (width 0.381) (layer F.Cu) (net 3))
 (segment (start 147.32 101.7651) (end 144.6751 104.41) (width 0.381) (layer F.Cu) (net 3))
 (segment (start 147.32 100.33) (end 147.32 101.7651) (width 0.381) (layer F.Cu) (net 3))
 (segment (start 139.599 106.68) (end 139.1 106.68) (width 0.381) (layer F.Cu) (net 3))
 (segment (start 141.869 104.41) (end 139.599 106.68) (width 0.381) (layer F.Cu) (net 3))
 (segment (start 142.875 104.41) (end 141.869 104.41) (width 0.381) (layer F.Cu) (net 3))
 (segment (start 125.722099 86.427901) (end 125.73 86.42) (width 0.381) (layer F.Cu) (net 4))
 (segment (start 125.722099 91.408099) (end 125.722099 86.427901) (width 0.381) (layer F.Cu) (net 4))
 (segment (start 126.389 92.075) (end 125.722099 91.408099) (width 0.381) (layer F.Cu) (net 4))
 (segment (start 124.375 86.42) (end 125.73 86.42) (width 0.381) (layer F.Cu) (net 4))
 (segment (start 127.27 92.075) (end 126.389 92.075) (width 0.381) (layer F.Cu) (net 4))
 (segment (start 125.73 86.42) (end 126.915 86.42) (width 0.381) (layer F.Cu) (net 4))
 (segment (start 128.151 103.048) (end 128.151 93.081) (width 0.381) (layer F.Cu) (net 4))
 (segment (start 127.27 92.2) (end 127.27 92.075) (width 0.381) (layer F.Cu) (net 4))
 (segment (start 128.151 93.081) (end 127.27 92.2) (width 0.381) (layer F.Cu) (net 4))
 (segment (start 127.6 103.599) (end 128.151 103.048) (width 0.381) (layer F.Cu) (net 4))
 (segment (start 127.6 106.68) (end 127.6 103.599) (width 0.381) (layer F.Cu) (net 4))
 (segment (start 147.32 112.125) (end 147.59 112.395) (width 0.381) (layer F.Cu) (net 5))
 (segment (start 147.32 110.49) (end 147.32 112.125) (width 0.381) (layer F.Cu) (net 5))
 (segment (start 136.845 97.49) (end 136.545 97.79) (width 0.381) (layer F.Cu) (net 11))
 (segment (start 136.845 95.885) (end 136.845 97.49) (width 0.381) (layer F.Cu) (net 11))
 (segment (start 134.308748 95.885) (end 136.114 95.885) (width 0.381) (layer F.Cu) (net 11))
 (segment (start 136.114 95.885) (end 136.845 95.885) (width 0.381) (layer F.Cu) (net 11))
 (segment (start 133.35 96.843748) (end 134.308748 95.885) (width 0.381) (layer F.Cu) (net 11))
 (segment (start 133.35 97.318748) (end 133.35 96.843748) (width 0.381) (layer F.Cu) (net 11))
 (segment (start 139.445 95.185) (end 138.745 95.885) (width 0.381) (layer F.Cu) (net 10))
 (segment (start 139.445 93.98) (end 139.445 95.185) (width 0.381) (layer F.Cu) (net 10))
 (segment (start 165.1 97.535) (end 165.1 98.745) (width 0.381) (layer F.Cu) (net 12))
 (segment (start 156.21 92.39) (end 156.21 91.915) (width 0.381) (layer F.Cu) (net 14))
 (segment (start 157.8 93.98) (end 156.21 92.39) (width 0.381) (layer F.Cu) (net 14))
 (segment (start 159.07 93.98) (end 157.8 93.98) (width 0.381) (layer F.Cu) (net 14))
 (segment (start 156.545001 87.269999) (end 157.395 86.42) (width 0.381) (layer F.Cu) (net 14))
 (segment (start 156.202099 87.612901) (end 156.545001 87.269999) (width 0.381) (layer F.Cu) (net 14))
 (segment (start 156.202099 90.751099) (end 156.202099 87.612901) (width 0.381) (layer F.Cu) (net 14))
 (segment (start 156.21 90.759) (end 156.202099 90.751099) (width 0.381) (layer F.Cu) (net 14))
 (segment (start 156.21 91.915) (end 156.21 90.759) (width 0.381) (layer F.Cu) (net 14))
 (segment (start 157.64 92.075) (end 157.48 91.915) (width 0.381) (layer F.Cu) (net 15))
 (segment (start 159.07 92.075) (end 157.64 92.075) (width 0.381) (layer F.Cu) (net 15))
 (segment (start 157.395 91.83) (end 157.48 91.915) (width 0.381) (layer F.Cu) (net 15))
 (segment (start 157.395 88.96) (end 157.395 91.83) (width 0.381) (layer F.Cu) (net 15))
 (segment (start 160.97 92.075) (end 160.97 93.98) (width 0.381) (layer F.Cu) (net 8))
 (segment (start 153.51 92.075) (end 153.67 91.915) (width 0.381) (layer F.Cu) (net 8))
 (segment (start 151.13 92.075) (end 144.78 92.075) (width 0.381) (layer F.Cu) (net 8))
 (segment (start 144.78 92.075) (end 138.745 92.075) (width 0.381) (layer F.Cu) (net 8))
 (segment (start 144.695 91.99) (end 144.78 92.075) (width 0.381) (layer F.Cu) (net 8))
 (segment (start 144.695 88.96) (end 144.695 91.99) (width 0.381) (layer F.Cu) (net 8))
 (via (at 152.4 92.075) (size 0.508) (drill 0.254) (layers F.Cu B.Cu) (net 8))
 (segment (start 152.4 92.075) (end 153.51 92.075) (width 0.381) (layer F.Cu) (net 8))
 (segment (start 151.13 92.075) (end 152.4 92.075) (width 0.381) (layer F.Cu) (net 8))
 (via (at 161.925 92.075) (size 0.508) (drill 0.254) (layers F.Cu B.Cu) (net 8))
 (segment (start 152.4 92.075) (end 161.925 92.075) (width 0.381) (layer B.Cu) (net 8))
 (segment (start 161.925 92.075) (end 160.97 92.075) (width 0.381) (layer F.Cu) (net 8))
 (segment (start 143.845001 89.809999) (end 144.695 88.96) (width 0.381) (layer B.Cu) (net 8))
 (segment (start 143.502099 90.152901) (end 143.845001 89.809999) (width 0.381) (layer B.Cu) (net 8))
 (segment (start 125.567901 90.152901) (end 143.502099 90.152901) (width 0.381) (layer B.Cu) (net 8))
 (segment (start 124.375 88.96) (end 125.567901 90.152901) (width 0.381) (layer B.Cu) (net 8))
 (segment (start 133.342099 90.754847) (end 133.342099 85.732901) (width 0.381) (layer F.Cu) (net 18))
 (segment (start 133.35 91.918748) (end 133.35 90.762748) (width 0.381) (layer F.Cu) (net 18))
 (segment (start 133.35 90.762748) (end 133.342099 90.754847) (width 0.381) (layer F.Cu) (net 18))
 (segment (start 136.225001 85.570001) (end 137.075 86.42) (width 0.381) (layer F.Cu) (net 18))
 (segment (start 135.882099 85.227099) (end 136.225001 85.570001) (width 0.381) (layer F.Cu) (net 18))
 (segment (start 133.847901 85.227099) (end 135.882099 85.227099) (width 0.381) (layer F.Cu) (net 18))
 (segment (start 133.342099 85.732901) (end 133.847901 85.227099) (width 0.381) (layer F.Cu) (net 18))
 (segment (start 136.688748 91.918748) (end 136.845 92.075) (width 0.381) (layer F.Cu) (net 9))
 (segment (start 135.727901 91.756649) (end 135.89 91.918748) (width 0.381) (layer F.Cu) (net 9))
 (segment (start 134.535 86.42) (end 135.727901 87.612901) (width 0.381) (layer F.Cu) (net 9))
 (segment (start 134.62 91.918748) (end 135.89 91.918748) (width 0.381) (layer F.Cu) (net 9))
 (segment (start 135.727901 87.612901) (end 135.727901 91.756649) (width 0.381) (layer F.Cu) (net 9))
 (segment (start 135.89 91.918748) (end 136.688748 91.918748) (width 0.381) (layer F.Cu) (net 9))
 (segment (start 130.802099 87.612901) (end 131.145001 87.269999) (width 0.381) (layer F.Cu) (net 19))
 (segment (start 130.802099 90.754847) (end 130.802099 87.612901) (width 0.381) (layer F.Cu) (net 19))
 (segment (start 131.145001 87.269999) (end 131.995 86.42) (width 0.381) (layer F.Cu) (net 19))
 (segment (start 130.81 90.762748) (end 130.802099 90.754847) (width 0.381) (layer F.Cu) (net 19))
 (segment (start 130.81 91.918748) (end 130.81 90.762748) (width 0.381) (layer F.Cu) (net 19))
 (segment (start 122.265 96.241) (end 122.265 103.035) (width 0.381) (layer F.Cu) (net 6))
 (segment (start 122.265 95.085) (end 122.265 96.241) (width 0.381) (layer F.Cu) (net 6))
 (segment (start 122.265 95.085) (end 127.155 95.085) (width 0.381) (layer F.Cu) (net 6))
 (segment (start 127.32 97.155) (end 127.32 95.25) (width 0.381) (layer F.Cu) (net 6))
 (segment (start 127.155 95.085) (end 127.32 95.25) (width 0.381) (layer F.Cu) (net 6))
 (segment (start 127.32 95.25) (end 127.32 94.615) (width 0.381) (layer F.Cu) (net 6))
 (segment (start 129.951 94.615) (end 132.08 92.486) (width 0.381) (layer F.Cu) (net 7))
 (segment (start 132.08 92.486) (end 132.08 91.918748) (width 0.381) (layer F.Cu) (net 7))
 (segment (start 129.22 94.615) (end 129.951 94.615) (width 0.381) (layer F.Cu) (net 7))
 (segment (start 165.1 100.645) (end 165.1 101.87) (width 0.381) (layer F.Cu) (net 13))
 (segment (start 132.08 97.318748) (end 132.08 99.06) (width 0.381) (layer F.Cu) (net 13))
 (via (at 145.41499 99.695) (size 0.508) (drill 0.254) (layers F.Cu B.Cu) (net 13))
 (segment (start 132.715 99.695) (end 145.05578 99.695) (width 0.381) (layer F.Cu) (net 13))
 (segment (start 145.05578 99.695) (end 145.41499 99.695) (width 0.381) (layer F.Cu) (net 13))
 (segment (start 132.08 99.06) (end 132.715 99.695) (width 0.381) (layer F.Cu) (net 13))
 (via (at 166.37002 99.695) (size 0.508) (drill 0.254) (layers F.Cu B.Cu) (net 13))
 (segment (start 145.41499 99.695) (end 166.37002 99.695) (width 0.381) (layer B.Cu) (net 13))
 (segment (start 165.4 100.645) (end 166.35 99.695) (width 0.381) (layer F.Cu) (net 13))
 (segment (start 166.35 99.695) (end 166.37002 99.695) (width 0.381) (layer F.Cu) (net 13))
 (segment (start 165.1 100.645) (end 165.4 100.645) (width 0.381) (layer F.Cu) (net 13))
 (segment (start 166.624019 99.441001) (end 166.37002 99.695) (width 0.381) (layer B.Cu) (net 13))
 (segment (start 167.00502 99.06) (end 166.624019 99.441001) (width 0.381) (layer B.Cu) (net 13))
 (segment (start 175.26 99.06) (end 167.00502 99.06) (width 0.381) (layer B.Cu) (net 13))
 (segment (start 154.94 92.39) (end 154.94 91.915) (width 0.381) (layer F.Cu) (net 16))
 (segment (start 151.13 96.2) (end 154.94 92.39) (width 0.381) (layer F.Cu) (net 16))
 (segment (start 151.13 97.155) (end 151.13 96.2) (width 0.381) (layer F.Cu) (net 16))
 (segment (start 135.759251 98.932999) (end 134.62 97.793748) (width 0.381) (layer F.Cu) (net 17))
 (segment (start 148.089621 98.932999) (end 135.759251 98.932999) (width 0.381) (layer F.Cu) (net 17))
 (segment (start 157.48 110.49) (end 157.48 108.323378) (width 0.381) (layer F.Cu) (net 17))
 (segment (start 134.62 97.793748) (end 134.62 97.318748) (width 0.381) (layer F.Cu) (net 17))
 (segment (start 157.48 108.323378) (end 148.089621 98.932999) (width 0.381) (layer F.Cu) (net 17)))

